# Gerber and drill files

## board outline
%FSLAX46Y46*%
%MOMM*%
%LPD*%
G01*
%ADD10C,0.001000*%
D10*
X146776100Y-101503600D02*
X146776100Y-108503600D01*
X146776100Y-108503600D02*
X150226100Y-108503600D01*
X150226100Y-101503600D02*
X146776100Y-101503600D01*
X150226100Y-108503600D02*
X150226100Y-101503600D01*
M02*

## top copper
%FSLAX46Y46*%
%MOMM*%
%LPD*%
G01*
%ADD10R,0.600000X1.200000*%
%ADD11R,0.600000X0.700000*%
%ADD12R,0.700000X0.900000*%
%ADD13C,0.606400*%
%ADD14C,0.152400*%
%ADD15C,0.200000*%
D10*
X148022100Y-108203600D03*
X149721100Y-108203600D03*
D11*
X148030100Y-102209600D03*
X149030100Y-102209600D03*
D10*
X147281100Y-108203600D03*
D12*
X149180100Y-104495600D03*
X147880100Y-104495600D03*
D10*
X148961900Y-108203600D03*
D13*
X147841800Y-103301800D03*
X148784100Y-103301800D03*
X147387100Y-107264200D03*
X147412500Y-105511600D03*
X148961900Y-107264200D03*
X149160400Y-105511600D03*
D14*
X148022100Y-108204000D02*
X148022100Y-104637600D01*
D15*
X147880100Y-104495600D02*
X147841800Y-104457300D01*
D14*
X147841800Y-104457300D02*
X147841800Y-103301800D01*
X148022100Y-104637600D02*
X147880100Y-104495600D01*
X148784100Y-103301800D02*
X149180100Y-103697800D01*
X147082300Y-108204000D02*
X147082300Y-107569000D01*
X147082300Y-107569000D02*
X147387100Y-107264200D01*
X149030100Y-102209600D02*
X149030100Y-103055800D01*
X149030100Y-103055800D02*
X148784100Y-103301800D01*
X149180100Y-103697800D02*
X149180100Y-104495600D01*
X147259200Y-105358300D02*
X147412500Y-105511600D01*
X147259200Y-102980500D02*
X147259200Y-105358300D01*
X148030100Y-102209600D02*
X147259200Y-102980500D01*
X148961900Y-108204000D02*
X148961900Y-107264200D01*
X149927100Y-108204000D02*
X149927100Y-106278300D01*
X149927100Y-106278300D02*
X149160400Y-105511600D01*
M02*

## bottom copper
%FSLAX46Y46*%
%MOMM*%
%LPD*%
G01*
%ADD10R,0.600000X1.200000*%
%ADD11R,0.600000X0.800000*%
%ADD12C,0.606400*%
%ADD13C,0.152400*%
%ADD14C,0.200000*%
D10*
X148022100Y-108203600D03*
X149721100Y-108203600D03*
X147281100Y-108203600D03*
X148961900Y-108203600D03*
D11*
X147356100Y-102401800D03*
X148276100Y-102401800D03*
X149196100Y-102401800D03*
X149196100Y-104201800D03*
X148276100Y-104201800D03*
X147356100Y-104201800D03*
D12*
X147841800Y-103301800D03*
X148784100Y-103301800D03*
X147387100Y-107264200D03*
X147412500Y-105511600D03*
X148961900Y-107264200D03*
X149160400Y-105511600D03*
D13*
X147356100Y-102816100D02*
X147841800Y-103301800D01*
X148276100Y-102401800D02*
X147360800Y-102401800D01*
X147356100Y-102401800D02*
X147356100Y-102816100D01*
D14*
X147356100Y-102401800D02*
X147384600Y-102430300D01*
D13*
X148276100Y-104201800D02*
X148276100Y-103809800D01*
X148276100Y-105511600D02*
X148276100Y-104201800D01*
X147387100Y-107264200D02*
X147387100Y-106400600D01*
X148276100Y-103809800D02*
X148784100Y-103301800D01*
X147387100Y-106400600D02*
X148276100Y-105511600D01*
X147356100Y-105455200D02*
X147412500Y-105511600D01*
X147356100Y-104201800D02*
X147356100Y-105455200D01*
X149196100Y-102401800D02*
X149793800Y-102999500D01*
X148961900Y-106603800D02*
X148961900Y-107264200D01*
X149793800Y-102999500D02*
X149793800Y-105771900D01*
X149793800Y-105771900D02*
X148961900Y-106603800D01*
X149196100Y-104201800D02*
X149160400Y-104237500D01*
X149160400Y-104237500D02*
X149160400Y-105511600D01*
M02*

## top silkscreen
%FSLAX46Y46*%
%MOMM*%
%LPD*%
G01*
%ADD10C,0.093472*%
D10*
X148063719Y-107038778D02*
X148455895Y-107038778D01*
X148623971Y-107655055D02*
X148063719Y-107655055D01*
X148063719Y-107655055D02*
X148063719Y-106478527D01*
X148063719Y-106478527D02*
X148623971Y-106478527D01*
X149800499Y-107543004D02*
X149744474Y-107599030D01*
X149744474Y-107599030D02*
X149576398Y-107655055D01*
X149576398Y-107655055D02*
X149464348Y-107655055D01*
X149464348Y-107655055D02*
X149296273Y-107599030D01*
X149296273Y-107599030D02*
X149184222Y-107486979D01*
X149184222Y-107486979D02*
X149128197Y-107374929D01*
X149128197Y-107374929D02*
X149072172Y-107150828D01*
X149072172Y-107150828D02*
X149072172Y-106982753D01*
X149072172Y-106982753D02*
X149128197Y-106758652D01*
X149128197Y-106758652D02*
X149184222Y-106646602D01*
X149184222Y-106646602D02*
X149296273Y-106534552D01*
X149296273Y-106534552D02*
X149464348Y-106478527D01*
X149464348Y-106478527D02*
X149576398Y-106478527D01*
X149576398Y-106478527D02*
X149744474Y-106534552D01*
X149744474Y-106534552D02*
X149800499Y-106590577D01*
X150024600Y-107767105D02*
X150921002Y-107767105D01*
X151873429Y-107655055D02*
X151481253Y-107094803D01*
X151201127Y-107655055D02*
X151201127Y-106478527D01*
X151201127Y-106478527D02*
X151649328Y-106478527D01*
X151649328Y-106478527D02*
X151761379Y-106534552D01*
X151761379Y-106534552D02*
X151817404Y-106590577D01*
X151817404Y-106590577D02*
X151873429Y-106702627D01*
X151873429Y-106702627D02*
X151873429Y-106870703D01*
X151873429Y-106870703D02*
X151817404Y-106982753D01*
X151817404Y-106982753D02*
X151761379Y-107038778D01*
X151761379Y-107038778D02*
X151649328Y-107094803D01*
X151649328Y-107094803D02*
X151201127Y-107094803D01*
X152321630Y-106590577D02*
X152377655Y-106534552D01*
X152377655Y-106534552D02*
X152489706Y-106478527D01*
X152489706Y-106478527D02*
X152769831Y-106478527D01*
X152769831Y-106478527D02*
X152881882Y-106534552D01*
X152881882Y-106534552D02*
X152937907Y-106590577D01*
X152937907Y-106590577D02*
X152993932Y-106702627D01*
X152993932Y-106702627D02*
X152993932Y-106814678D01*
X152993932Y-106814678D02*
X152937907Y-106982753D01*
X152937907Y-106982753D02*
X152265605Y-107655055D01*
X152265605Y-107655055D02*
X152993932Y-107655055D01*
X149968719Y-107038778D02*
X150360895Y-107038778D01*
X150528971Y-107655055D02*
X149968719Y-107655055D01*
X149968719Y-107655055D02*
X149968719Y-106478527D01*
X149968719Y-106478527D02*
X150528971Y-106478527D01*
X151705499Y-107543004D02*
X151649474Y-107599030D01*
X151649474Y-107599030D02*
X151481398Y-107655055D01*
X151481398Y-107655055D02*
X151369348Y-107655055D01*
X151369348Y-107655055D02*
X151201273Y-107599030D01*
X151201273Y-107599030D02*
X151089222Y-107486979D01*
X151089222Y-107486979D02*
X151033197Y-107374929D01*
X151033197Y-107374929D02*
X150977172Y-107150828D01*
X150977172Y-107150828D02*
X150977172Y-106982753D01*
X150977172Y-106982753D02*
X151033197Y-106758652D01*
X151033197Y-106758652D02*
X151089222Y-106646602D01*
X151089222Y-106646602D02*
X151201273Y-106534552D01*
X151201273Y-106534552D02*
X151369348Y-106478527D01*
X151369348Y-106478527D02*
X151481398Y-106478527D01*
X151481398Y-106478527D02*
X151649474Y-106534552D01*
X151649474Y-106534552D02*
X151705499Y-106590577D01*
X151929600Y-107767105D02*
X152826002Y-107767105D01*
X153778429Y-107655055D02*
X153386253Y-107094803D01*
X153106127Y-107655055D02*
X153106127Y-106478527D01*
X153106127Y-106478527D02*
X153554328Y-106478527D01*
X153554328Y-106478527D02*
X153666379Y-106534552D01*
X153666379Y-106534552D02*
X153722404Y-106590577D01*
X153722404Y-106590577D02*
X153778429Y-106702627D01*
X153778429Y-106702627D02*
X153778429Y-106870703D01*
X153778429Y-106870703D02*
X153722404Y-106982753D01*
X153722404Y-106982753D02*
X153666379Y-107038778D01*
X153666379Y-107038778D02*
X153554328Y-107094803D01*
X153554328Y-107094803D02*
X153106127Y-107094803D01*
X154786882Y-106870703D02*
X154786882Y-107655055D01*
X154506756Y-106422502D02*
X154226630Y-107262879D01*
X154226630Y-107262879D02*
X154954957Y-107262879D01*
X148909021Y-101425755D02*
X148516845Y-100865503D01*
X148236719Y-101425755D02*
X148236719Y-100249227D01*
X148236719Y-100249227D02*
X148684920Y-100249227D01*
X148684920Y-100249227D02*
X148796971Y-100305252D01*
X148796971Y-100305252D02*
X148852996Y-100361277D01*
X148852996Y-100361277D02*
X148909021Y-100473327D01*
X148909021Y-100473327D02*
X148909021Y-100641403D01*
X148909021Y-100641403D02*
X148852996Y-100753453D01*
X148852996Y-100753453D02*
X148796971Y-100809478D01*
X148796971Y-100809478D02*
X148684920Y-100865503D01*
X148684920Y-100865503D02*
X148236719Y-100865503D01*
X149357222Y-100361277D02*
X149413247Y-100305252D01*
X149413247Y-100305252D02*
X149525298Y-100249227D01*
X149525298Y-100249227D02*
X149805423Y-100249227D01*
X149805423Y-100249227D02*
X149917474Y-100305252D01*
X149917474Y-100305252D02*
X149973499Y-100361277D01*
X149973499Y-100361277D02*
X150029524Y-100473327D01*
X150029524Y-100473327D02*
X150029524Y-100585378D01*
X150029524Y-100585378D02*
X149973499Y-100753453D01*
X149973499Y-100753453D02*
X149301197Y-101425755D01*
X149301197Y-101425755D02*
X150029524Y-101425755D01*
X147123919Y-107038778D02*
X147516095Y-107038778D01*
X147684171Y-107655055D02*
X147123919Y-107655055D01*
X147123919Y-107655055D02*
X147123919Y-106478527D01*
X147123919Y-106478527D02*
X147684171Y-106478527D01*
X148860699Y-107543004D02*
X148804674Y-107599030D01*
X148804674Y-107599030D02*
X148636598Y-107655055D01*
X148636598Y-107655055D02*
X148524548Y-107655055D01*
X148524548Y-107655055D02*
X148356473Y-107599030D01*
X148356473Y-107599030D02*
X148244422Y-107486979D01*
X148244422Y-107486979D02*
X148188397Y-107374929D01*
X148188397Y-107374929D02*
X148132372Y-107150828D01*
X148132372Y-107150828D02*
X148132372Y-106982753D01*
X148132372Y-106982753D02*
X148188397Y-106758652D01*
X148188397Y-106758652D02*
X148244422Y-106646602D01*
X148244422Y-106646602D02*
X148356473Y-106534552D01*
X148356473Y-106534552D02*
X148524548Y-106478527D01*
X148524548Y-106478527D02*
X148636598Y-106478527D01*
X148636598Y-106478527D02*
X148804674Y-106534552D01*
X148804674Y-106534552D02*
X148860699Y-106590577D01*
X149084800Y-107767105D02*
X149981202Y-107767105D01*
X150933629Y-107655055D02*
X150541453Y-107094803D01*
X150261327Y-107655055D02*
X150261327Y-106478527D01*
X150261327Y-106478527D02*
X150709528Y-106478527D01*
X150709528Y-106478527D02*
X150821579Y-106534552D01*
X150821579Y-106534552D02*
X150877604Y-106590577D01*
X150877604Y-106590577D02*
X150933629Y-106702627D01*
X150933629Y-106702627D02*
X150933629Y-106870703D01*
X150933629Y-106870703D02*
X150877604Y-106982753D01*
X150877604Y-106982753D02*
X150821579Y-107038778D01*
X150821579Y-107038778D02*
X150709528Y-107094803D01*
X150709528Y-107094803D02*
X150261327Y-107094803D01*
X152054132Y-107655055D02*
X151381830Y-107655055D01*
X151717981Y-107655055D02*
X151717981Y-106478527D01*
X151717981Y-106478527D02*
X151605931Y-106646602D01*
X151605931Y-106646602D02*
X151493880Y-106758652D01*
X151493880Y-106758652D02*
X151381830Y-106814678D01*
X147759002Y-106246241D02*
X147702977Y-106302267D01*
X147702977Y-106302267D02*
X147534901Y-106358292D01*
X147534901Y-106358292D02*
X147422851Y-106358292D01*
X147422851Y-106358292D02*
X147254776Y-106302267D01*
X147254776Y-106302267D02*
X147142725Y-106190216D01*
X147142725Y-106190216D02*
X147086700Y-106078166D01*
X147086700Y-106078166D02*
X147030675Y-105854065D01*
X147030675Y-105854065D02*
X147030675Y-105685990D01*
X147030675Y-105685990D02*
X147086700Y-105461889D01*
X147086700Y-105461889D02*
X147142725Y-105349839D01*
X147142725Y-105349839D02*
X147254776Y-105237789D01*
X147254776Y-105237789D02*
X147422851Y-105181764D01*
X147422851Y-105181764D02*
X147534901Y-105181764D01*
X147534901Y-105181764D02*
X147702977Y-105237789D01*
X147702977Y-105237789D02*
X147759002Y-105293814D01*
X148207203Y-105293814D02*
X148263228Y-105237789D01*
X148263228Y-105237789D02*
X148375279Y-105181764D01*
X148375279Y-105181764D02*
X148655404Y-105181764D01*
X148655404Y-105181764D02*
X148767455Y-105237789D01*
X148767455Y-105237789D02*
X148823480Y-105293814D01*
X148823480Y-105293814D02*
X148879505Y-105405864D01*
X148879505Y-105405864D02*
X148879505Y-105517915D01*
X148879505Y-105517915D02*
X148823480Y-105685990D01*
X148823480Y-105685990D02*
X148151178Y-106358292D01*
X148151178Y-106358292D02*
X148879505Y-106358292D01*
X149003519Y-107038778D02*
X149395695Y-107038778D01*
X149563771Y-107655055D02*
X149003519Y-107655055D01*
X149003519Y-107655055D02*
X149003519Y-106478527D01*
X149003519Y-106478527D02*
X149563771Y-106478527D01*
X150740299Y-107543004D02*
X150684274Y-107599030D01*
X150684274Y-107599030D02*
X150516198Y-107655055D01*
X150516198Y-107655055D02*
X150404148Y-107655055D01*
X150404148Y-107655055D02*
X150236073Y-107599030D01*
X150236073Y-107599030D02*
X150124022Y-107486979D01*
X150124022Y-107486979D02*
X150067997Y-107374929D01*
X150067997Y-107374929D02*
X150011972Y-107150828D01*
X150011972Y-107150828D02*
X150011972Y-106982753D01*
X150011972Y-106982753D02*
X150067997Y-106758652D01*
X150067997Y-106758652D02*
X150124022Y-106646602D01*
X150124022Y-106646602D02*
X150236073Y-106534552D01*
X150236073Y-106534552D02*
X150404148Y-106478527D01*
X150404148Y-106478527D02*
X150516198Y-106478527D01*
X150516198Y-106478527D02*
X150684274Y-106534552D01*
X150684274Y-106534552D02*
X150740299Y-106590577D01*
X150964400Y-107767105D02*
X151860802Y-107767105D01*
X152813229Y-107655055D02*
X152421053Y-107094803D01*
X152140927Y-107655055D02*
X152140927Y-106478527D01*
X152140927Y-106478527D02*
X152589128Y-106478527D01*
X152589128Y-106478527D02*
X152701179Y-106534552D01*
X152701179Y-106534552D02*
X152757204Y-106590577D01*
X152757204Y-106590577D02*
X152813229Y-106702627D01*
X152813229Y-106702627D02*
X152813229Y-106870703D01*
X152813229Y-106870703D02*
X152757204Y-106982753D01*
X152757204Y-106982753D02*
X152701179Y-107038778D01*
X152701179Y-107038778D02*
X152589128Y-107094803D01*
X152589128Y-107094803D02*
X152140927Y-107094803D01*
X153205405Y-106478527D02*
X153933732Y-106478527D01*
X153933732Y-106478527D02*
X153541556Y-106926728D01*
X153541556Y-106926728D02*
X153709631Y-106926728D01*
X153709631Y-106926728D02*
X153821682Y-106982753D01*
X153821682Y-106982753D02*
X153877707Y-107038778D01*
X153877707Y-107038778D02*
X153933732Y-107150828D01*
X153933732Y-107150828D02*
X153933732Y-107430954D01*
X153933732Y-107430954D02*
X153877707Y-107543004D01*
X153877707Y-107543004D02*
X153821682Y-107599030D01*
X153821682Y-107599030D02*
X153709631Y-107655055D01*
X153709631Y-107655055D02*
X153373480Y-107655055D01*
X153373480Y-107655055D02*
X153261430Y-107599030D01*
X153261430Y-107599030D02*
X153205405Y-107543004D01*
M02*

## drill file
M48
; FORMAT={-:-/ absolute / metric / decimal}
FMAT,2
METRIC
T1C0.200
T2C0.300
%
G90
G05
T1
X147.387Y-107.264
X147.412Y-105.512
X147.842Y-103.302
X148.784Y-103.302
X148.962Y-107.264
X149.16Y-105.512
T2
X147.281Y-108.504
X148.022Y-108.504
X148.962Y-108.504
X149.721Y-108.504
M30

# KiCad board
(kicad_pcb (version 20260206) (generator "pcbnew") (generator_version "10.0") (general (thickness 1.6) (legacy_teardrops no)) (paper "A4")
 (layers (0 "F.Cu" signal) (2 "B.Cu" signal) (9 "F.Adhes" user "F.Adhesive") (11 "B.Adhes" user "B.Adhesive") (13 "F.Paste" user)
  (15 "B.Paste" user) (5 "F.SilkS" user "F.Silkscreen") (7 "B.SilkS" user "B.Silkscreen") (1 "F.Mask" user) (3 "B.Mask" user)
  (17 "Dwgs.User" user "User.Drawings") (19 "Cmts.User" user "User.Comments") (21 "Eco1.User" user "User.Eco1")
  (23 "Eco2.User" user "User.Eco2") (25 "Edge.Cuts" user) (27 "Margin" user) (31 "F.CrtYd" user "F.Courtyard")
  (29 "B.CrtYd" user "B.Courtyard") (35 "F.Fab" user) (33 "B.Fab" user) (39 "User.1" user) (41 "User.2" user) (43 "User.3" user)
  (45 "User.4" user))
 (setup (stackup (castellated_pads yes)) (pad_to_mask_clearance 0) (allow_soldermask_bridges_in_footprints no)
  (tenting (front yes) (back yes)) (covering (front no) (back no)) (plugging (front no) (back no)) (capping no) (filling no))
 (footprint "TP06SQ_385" (layer "F.Cu") (at 148.0221 108.204)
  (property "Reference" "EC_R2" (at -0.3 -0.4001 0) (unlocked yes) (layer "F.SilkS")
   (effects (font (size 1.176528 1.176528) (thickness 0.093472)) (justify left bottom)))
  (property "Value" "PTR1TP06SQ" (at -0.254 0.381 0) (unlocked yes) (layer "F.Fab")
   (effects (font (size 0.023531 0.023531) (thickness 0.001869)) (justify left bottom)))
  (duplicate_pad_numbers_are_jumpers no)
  (pad "TP" thru_hole rect (at 0 0.2996) (size 0.6 1.2) (drill 0.3 (offset 0 -0.3000)) (layers "*.Cu" "*.Mask") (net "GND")
   (solder_mask_margin 0) (solder_paste_margin 0) (thermal_bridge_angle 0)))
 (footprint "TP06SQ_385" (layer "F.Cu") (at 149.9271 108.204)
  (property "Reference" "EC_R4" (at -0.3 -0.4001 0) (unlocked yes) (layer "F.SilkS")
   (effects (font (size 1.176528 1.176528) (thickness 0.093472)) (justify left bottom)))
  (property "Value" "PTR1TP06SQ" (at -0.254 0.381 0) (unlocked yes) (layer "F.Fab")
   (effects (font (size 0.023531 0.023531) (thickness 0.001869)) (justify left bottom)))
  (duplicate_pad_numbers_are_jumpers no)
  (pad "TP" thru_hole rect (at -0.2060 0.2996) (size 0.6 1.2) (drill 0.3 (offset 0 -0.3000)) (layers "*.Cu" "*.Mask") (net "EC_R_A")
   (solder_mask_margin 0) (solder_paste_margin 0) (thermal_bridge_angle 0)))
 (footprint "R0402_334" (layer "F.Cu") (at 148.5301 102.2096)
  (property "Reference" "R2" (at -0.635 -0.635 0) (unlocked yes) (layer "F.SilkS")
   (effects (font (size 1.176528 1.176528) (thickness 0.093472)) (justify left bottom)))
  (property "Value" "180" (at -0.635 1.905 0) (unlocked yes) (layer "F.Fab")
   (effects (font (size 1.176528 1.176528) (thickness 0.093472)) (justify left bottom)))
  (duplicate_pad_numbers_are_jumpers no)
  (pad "1" smd rect (at -0.5 0) (size 0.6 0.7) (layers "F.Cu" "F.Mask" "F.Paste") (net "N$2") (solder_mask_margin 0.1016)
   (solder_paste_margin 0) (thermal_bridge_angle 0))
  (pad "2" smd rect (at 0.5 0) (size 0.6 0.7) (layers "F.Cu" "F.Mask" "F.Paste") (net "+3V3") (solder_mask_margin 0.1016)
   (solder_paste_margin 0) (thermal_bridge_angle 0)))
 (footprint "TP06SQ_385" (layer "F.Cu") (at 147.0823 108.204)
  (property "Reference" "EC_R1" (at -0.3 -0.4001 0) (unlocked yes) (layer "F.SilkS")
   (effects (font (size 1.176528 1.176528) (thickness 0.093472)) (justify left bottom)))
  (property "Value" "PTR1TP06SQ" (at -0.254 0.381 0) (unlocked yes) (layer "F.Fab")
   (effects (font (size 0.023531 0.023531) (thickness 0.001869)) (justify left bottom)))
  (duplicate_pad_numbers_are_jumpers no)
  (pad "TP" thru_hole rect (at 0.1988 0.2996) (size 0.6 1.2) (drill 0.3 (offset 0 -0.3000)) (layers "*.Cu" "*.Mask") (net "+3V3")
   (solder_mask_margin 0) (solder_paste_margin 0) (thermal_bridge_angle 0)))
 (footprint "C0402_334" (layer "F.Cu") (at 148.5301 104.4956 180)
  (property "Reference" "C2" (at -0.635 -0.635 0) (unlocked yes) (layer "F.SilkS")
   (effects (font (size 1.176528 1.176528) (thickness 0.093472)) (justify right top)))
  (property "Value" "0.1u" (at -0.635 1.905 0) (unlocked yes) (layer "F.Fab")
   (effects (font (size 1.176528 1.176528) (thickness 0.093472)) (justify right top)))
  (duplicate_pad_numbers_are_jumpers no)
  (pad "1" smd rect (at -0.65 0 180) (size 0.7 0.9) (layers "F.Cu" "F.Mask" "F.Paste") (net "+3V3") (solder_mask_margin 0.1016)
   (solder_paste_margin 0) (thermal_bridge_angle 0))
  (pad "2" smd rect (at 0.65 0 180) (size 0.7 0.9) (layers "F.Cu" "F.Mask" "F.Paste") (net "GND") (solder_mask_margin 0.1016)
   (solder_paste_margin 0) (thermal_bridge_angle 0)))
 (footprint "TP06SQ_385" (layer "F.Cu") (at 148.9619 108.204)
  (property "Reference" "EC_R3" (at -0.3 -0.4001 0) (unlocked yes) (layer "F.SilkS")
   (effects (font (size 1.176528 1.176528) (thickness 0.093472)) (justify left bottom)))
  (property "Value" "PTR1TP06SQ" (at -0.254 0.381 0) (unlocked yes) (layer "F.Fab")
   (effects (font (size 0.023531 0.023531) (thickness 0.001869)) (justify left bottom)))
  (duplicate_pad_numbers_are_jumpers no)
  (pad "TP" thru_hole rect (at 0 0.2996) (size 0.6 1.2) (drill 0.3 (offset 0 -0.3000)) (layers "*.Cu" "*.Mask") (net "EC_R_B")
   (solder_mask_margin 0) (solder_paste_margin 0) (thermal_bridge_angle 0)))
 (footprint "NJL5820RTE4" (layer "B.Cu") (at 148.2761 103.3018)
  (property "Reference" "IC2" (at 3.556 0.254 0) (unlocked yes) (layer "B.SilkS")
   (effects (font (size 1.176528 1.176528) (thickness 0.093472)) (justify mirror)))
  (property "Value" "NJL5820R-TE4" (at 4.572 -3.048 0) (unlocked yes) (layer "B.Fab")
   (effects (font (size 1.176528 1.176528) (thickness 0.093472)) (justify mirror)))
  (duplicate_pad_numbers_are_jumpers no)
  (pad "1" smd rect (at -0.92 -0.9 270) (size 0.8 0.6) (layers "B.Cu" "B.Mask" "B.Paste") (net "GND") (solder_mask_margin 0.1016)
   (solder_paste_margin 0) (thermal_bridge_angle 0))
  (pad "2" smd rect (at 0 -0.9 270) (size 0.8 0.6) (layers "B.Cu" "B.Mask" "B.Paste") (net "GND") (solder_mask_margin 0.1016)
   (solder_paste_margin 0) (thermal_bridge_angle 0))
  (pad "3" smd rect (at 0.92 -0.9 270) (size 0.8 0.6) (layers "B.Cu" "B.Mask" "B.Paste") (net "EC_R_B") (solder_mask_margin 0.1016)
   (solder_paste_margin 0) (thermal_bridge_angle 0))
  (pad "4" smd rect (at 0.92 0.9 270) (size 0.8 0.6) (layers "B.Cu" "B.Mask" "B.Paste") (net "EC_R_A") (solder_mask_margin 0.1016)
   (solder_paste_margin 0) (thermal_bridge_angle 0))
  (pad "5" smd rect (at 0 0.9 270) (size 0.8 0.6) (layers "B.Cu" "B.Mask" "B.Paste") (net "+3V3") (solder_mask_margin 0.1016)
   (solder_paste_margin 0) (thermal_bridge_angle 0))
  (pad "6" smd rect (at -0.92 0.9 270) (size 0.8 0.6) (layers "B.Cu" "B.Mask" "B.Paste") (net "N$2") (solder_mask_margin 0.1016)
   (solder_paste_margin 0) (thermal_bridge_angle 0)))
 (gr_line (start 146.7761 101.5036) (end 146.7761 108.5036) (stroke (width 0.001) (type solid)) (layer "Edge.Cuts"))
 (gr_line (start 146.7761 108.5036) (end 150.2261 108.5036) (stroke (width 0.001) (type solid)) (layer "Edge.Cuts"))
 (gr_line (start 150.2261 101.5036) (end 146.7761 101.5036) (stroke (width 0.001) (type solid)) (layer "Edge.Cuts"))
 (gr_line (start 150.2261 108.5036) (end 150.2261 101.5036) (stroke (width 0.001) (type solid)) (layer "Edge.Cuts"))
 (segment (start 148.0221 108.204) (end 148.0221 104.6376) (width 0.1524) (layer "F.Cu") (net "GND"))
 (segment (start 147.8801 104.4956) (end 147.8418 104.4573) (width 0.2) (layer "F.Cu") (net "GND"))
 (segment (start 147.8418 104.4573) (end 147.8418 103.3018) (width 0.1524) (layer "F.Cu") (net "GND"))
 (segment (start 148.0221 104.6376) (end 147.8801 104.4956) (width 0.1524) (layer "F.Cu") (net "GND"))
 (via (at 147.8418 103.3018) (size 0.6064) (drill 0.2) (layers "F.Cu" "B.Cu") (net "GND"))
 (segment (start 147.3561 102.8161) (end 147.8418 103.3018) (width 0.1524) (layer "B.Cu") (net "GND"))
 (segment (start 148.2761 102.4018) (end 147.3608 102.4018) (width 0.1524) (layer "B.Cu") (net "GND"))
 (segment (start 147.3561 102.4018) (end 147.3561 102.8161) (width 0.1524) (layer "B.Cu") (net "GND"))
 (segment (start 147.3561 102.4018) (end 147.3846 102.4303) (width 0.2) (layer "B.Cu") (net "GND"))
 (segment (start 148.7841 103.3018) (end 149.1801 103.6978) (width 0.1524) (layer "F.Cu") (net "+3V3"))
 (segment (start 147.0823 108.204) (end 147.0823 107.569) (width 0.1524) (layer "F.Cu") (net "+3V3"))
 (segment (start 147.0823 107.569) (end 147.3871 107.2642) (width 0.1524) (layer "F.Cu") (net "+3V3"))
 (segment (start 149.0301 102.2096) (end 149.0301 103.0558) (width 0.1524) (layer "F.Cu") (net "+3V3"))
 (segment (start 149.0301 103.0558) (end 148.7841 103.3018) (width 0.1524) (layer "F.Cu") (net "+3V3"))
 (segment (start 149.1801 103.6978) (end 149.1801 104.4956) (width 0.1524) (layer "F.Cu") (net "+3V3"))
 (via (at 148.7841 103.3018) (size 0.6064) (drill 0.2) (layers "F.Cu" "B.Cu") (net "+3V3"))
 (via (at 147.3871 107.2642) (size 0.6064) (drill 0.2) (layers "F.Cu" "B.Cu") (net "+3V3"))
 (segment (start 148.2761 104.2018) (end 148.2761 103.8098) (width 0.1524) (layer "B.Cu") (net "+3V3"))
 (segment (start 148.2761 105.5116) (end 148.2761 104.2018) (width 0.1524) (layer "B.Cu") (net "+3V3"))
 (segment (start 147.3871 107.2642) (end 147.3871 106.4006) (width 0.1524) (layer "B.Cu") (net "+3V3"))
 (segment (start 148.2761 103.8098) (end 148.7841 103.3018) (width 0.1524) (layer "B.Cu") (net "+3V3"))
 (segment (start 147.3871 106.4006) (end 148.2761 105.5116) (width 0.1524) (layer "B.Cu") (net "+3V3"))
 (segment (start 147.2592 105.3583) (end 147.4125 105.5116) (width 0.1524) (layer "F.Cu") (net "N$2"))
 (segment (start 147.2592 102.9805) (end 147.2592 105.3583) (width 0.1524) (layer "F.Cu") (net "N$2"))
 (segment (start 148.0301 102.2096) (end 147.2592 102.9805) (width 0.1524) (layer "F.Cu") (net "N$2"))
 (via (at 147.4125 105.5116) (size 0.6064) (drill 0.2) (layers "F.Cu" "B.Cu") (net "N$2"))
 (segment (start 147.3561 105.4552) (end 147.4125 105.5116) (width 0.1524) (layer "B.Cu") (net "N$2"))
 (segment (start 147.3561 104.2018) (end 147.3561 105.4552) (width 0.1524) (layer "B.Cu") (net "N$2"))
 (segment (start 148.9619 108.204) (end 148.9619 107.2642) (width 0.1524) (layer "F.Cu") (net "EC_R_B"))
 (via (at 148.9619 107.2642) (size 0.6064) (drill 0.2) (layers "F.Cu" "B.Cu") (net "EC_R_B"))
 (segment (start 149.1961 102.4018) (end 149.7938 102.9995) (width 0.1524) (layer "B.Cu") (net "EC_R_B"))
 (segment (start 148.9619 106.6038) (end 148.9619 107.2642) (width 0.1524) (layer "B.Cu") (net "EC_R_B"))
 (segment (start 149.7938 102.9995) (end 149.7938 105.7719) (width 0.1524) (layer "B.Cu") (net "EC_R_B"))
 (segment (start 149.7938 105.7719) (end 148.9619 106.6038) (width 0.1524) (layer "B.Cu") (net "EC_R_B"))
 (segment (start 149.9271 108.204) (end 149.9271 106.2783) (width 0.1524) (layer "F.Cu") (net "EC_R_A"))
 (segment (start 149.9271 106.2783) (end 149.1604 105.5116) (width 0.1524) (layer "F.Cu") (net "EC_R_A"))
 (via (at 149.1604 105.5116) (size 0.6064) (drill 0.2) (layers "F.Cu" "B.Cu") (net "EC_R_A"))
 (segment (start 149.1961 104.2018) (end 149.1604 104.2375) (width 0.1524) (layer "B.Cu") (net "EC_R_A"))
 (segment (start 149.1604 104.2375) (end 149.1604 105.5116) (width 0.1524) (layer "B.Cu") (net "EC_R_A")))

